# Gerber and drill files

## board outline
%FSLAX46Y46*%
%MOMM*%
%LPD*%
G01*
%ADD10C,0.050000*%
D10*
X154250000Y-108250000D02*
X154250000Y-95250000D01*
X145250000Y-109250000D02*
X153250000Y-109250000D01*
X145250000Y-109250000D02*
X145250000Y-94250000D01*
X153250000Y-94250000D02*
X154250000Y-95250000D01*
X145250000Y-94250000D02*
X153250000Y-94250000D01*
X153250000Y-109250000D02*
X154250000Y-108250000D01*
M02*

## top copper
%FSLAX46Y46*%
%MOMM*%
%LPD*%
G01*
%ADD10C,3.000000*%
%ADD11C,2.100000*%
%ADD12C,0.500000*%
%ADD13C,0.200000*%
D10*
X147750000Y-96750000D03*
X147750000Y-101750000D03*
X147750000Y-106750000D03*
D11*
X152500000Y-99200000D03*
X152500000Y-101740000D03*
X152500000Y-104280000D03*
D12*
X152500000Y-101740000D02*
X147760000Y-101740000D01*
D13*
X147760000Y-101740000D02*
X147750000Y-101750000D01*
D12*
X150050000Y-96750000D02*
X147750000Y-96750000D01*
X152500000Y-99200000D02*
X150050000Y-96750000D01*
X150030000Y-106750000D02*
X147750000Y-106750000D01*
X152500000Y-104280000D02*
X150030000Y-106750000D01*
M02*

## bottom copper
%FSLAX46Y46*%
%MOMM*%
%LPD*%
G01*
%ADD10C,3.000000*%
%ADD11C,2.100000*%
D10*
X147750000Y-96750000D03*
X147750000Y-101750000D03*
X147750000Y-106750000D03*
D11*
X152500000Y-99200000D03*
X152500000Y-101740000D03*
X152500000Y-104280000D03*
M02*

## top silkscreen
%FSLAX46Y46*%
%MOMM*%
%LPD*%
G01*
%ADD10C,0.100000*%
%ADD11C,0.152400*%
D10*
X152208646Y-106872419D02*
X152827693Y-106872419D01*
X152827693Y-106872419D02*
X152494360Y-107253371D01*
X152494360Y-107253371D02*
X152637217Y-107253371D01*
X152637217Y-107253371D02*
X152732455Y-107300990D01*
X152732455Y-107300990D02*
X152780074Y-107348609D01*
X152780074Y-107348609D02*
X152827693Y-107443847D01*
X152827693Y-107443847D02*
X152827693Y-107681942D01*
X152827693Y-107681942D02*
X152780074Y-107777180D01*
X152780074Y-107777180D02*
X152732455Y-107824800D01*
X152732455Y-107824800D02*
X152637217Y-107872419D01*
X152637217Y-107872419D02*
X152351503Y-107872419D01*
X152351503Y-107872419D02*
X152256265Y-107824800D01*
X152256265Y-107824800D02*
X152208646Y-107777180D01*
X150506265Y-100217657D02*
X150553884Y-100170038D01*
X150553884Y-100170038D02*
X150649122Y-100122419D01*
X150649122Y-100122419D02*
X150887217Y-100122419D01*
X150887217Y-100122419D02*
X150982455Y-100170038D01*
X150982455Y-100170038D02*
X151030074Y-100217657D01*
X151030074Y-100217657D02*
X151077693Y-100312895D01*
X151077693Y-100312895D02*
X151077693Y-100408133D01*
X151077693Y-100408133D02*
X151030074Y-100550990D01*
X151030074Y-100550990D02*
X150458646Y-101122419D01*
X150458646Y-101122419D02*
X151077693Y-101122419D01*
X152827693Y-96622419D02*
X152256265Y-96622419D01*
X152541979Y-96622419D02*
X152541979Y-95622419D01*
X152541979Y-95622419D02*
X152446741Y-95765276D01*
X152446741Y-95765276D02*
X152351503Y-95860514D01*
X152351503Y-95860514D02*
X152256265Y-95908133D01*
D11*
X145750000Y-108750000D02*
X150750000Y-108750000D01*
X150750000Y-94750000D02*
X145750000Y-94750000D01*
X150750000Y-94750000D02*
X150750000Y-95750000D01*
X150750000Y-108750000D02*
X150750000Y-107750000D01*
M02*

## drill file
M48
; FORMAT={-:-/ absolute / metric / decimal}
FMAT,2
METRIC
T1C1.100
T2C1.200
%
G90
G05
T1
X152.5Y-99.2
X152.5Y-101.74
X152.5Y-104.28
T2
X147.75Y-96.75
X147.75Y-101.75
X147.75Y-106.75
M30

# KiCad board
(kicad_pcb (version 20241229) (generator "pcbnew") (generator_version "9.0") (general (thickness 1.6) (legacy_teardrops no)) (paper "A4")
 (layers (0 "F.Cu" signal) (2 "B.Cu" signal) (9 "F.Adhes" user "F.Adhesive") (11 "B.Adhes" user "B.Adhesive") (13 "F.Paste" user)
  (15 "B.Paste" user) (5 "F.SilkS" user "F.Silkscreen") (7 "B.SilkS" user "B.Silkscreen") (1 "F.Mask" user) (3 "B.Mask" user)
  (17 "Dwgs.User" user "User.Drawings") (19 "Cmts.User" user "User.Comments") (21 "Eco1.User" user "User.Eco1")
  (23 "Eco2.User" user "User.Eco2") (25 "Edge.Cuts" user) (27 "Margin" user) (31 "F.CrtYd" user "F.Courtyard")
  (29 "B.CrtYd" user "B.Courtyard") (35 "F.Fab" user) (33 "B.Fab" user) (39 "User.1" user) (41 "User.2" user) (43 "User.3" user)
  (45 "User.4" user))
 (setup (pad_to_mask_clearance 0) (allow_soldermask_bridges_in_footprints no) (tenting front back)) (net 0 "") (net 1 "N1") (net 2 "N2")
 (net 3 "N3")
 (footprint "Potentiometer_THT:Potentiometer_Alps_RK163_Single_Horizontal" (layer "F.Cu") (at 147.75 96.75)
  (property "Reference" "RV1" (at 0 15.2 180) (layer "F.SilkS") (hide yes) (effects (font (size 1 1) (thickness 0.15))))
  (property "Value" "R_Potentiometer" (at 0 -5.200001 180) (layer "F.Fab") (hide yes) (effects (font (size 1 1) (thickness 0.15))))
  (fp_line (start -2 12) (end 3 12) (stroke (width 0.1524) (type solid)) (layer "F.SilkS"))
  (fp_line (start 3 -2) (end -2 -2) (stroke (width 0.1524) (type solid)) (layer "F.SilkS"))
  (fp_line (start 3 -2) (end 3 -1) (stroke (width 0.1524) (type solid)) (layer "F.SilkS"))
  (fp_line (start 3 12) (end 3 11) (stroke (width 0.1524) (type solid)) (layer "F.SilkS"))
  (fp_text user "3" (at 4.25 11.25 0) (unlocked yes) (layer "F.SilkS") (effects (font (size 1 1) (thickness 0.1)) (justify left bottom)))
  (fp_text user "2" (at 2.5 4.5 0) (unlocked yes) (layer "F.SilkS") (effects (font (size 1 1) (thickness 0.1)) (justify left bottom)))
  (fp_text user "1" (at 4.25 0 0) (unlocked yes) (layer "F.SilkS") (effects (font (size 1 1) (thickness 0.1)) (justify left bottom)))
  (pad "1" thru_hole circle (at 0 0 180) (size 3 3) (drill 1.2) (layers "*.Cu" "*.Mask") (remove_unused_layers no) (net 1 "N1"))
  (pad "2" thru_hole circle (at 0 5 180) (size 3 3) (drill 1.2) (layers "*.Cu" "*.Mask") (remove_unused_layers no) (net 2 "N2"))
  (pad "3" thru_hole circle (at 0 10 180) (size 3 3) (drill 1.2) (layers "*.Cu" "*.Mask") (remove_unused_layers no) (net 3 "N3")))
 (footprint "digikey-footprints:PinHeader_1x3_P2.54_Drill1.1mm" (layer "F.Cu") (at 152.5 99.2 -90)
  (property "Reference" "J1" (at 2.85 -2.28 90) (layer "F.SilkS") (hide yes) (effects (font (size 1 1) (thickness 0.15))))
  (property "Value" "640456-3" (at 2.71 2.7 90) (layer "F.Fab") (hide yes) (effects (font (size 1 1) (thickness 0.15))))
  (pad "1" thru_hole circle (at 0 0 270) (size 2.1 2.1) (drill 1.1) (layers "*.Cu" "*.Mask") (remove_unused_layers no) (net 1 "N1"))
  (pad "2" thru_hole circle (at 2.54 0 270) (size 2.1 2.1) (drill 1.1) (layers "*.Cu" "*.Mask") (remove_unused_layers no) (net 2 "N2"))
  (pad "3" thru_hole circle (at 5.08 0 270) (size 2.1 2.1) (drill 1.1) (layers "*.Cu" "*.Mask") (remove_unused_layers no) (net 3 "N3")))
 (gr_line (start 154.25 108.25) (end 154.25 95.25) (stroke (width 0.05) (type default)) (layer "Edge.Cuts"))
 (gr_line (start 145.25 109.25) (end 153.25 109.25) (stroke (width 0.05) (type default)) (layer "Edge.Cuts"))
 (gr_line (start 145.25 109.25) (end 145.25 94.25) (stroke (width 0.05) (type default)) (layer "Edge.Cuts"))
 (gr_line (start 153.25 94.25) (end 154.25 95.25) (stroke (width 0.05) (type default)) (layer "Edge.Cuts"))
 (gr_line (start 145.25 94.25) (end 153.25 94.25) (stroke (width 0.05) (type default)) (layer "Edge.Cuts"))
 (gr_line (start 153.25 109.25) (end 154.25 108.25) (stroke (width 0.05) (type default)) (layer "Edge.Cuts"))
 (segment (start 152.5 101.74) (end 147.76 101.74) (width 0.5) (layer "F.Cu") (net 2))
 (segment (start 147.76 101.74) (end 147.75 101.75) (width 0.2) (layer "F.Cu") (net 2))
 (segment (start 150.05 96.75) (end 147.75 96.75) (width 0.5) (layer "F.Cu") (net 1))
 (segment (start 152.5 99.2) (end 150.05 96.75) (width 0.5) (layer "F.Cu") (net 1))
 (segment (start 150.03 106.75) (end 147.75 106.75) (width 0.5) (layer "F.Cu") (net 3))
 (segment (start 152.5 104.28) (end 150.03 106.75) (width 0.5) (layer "F.Cu") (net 3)))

